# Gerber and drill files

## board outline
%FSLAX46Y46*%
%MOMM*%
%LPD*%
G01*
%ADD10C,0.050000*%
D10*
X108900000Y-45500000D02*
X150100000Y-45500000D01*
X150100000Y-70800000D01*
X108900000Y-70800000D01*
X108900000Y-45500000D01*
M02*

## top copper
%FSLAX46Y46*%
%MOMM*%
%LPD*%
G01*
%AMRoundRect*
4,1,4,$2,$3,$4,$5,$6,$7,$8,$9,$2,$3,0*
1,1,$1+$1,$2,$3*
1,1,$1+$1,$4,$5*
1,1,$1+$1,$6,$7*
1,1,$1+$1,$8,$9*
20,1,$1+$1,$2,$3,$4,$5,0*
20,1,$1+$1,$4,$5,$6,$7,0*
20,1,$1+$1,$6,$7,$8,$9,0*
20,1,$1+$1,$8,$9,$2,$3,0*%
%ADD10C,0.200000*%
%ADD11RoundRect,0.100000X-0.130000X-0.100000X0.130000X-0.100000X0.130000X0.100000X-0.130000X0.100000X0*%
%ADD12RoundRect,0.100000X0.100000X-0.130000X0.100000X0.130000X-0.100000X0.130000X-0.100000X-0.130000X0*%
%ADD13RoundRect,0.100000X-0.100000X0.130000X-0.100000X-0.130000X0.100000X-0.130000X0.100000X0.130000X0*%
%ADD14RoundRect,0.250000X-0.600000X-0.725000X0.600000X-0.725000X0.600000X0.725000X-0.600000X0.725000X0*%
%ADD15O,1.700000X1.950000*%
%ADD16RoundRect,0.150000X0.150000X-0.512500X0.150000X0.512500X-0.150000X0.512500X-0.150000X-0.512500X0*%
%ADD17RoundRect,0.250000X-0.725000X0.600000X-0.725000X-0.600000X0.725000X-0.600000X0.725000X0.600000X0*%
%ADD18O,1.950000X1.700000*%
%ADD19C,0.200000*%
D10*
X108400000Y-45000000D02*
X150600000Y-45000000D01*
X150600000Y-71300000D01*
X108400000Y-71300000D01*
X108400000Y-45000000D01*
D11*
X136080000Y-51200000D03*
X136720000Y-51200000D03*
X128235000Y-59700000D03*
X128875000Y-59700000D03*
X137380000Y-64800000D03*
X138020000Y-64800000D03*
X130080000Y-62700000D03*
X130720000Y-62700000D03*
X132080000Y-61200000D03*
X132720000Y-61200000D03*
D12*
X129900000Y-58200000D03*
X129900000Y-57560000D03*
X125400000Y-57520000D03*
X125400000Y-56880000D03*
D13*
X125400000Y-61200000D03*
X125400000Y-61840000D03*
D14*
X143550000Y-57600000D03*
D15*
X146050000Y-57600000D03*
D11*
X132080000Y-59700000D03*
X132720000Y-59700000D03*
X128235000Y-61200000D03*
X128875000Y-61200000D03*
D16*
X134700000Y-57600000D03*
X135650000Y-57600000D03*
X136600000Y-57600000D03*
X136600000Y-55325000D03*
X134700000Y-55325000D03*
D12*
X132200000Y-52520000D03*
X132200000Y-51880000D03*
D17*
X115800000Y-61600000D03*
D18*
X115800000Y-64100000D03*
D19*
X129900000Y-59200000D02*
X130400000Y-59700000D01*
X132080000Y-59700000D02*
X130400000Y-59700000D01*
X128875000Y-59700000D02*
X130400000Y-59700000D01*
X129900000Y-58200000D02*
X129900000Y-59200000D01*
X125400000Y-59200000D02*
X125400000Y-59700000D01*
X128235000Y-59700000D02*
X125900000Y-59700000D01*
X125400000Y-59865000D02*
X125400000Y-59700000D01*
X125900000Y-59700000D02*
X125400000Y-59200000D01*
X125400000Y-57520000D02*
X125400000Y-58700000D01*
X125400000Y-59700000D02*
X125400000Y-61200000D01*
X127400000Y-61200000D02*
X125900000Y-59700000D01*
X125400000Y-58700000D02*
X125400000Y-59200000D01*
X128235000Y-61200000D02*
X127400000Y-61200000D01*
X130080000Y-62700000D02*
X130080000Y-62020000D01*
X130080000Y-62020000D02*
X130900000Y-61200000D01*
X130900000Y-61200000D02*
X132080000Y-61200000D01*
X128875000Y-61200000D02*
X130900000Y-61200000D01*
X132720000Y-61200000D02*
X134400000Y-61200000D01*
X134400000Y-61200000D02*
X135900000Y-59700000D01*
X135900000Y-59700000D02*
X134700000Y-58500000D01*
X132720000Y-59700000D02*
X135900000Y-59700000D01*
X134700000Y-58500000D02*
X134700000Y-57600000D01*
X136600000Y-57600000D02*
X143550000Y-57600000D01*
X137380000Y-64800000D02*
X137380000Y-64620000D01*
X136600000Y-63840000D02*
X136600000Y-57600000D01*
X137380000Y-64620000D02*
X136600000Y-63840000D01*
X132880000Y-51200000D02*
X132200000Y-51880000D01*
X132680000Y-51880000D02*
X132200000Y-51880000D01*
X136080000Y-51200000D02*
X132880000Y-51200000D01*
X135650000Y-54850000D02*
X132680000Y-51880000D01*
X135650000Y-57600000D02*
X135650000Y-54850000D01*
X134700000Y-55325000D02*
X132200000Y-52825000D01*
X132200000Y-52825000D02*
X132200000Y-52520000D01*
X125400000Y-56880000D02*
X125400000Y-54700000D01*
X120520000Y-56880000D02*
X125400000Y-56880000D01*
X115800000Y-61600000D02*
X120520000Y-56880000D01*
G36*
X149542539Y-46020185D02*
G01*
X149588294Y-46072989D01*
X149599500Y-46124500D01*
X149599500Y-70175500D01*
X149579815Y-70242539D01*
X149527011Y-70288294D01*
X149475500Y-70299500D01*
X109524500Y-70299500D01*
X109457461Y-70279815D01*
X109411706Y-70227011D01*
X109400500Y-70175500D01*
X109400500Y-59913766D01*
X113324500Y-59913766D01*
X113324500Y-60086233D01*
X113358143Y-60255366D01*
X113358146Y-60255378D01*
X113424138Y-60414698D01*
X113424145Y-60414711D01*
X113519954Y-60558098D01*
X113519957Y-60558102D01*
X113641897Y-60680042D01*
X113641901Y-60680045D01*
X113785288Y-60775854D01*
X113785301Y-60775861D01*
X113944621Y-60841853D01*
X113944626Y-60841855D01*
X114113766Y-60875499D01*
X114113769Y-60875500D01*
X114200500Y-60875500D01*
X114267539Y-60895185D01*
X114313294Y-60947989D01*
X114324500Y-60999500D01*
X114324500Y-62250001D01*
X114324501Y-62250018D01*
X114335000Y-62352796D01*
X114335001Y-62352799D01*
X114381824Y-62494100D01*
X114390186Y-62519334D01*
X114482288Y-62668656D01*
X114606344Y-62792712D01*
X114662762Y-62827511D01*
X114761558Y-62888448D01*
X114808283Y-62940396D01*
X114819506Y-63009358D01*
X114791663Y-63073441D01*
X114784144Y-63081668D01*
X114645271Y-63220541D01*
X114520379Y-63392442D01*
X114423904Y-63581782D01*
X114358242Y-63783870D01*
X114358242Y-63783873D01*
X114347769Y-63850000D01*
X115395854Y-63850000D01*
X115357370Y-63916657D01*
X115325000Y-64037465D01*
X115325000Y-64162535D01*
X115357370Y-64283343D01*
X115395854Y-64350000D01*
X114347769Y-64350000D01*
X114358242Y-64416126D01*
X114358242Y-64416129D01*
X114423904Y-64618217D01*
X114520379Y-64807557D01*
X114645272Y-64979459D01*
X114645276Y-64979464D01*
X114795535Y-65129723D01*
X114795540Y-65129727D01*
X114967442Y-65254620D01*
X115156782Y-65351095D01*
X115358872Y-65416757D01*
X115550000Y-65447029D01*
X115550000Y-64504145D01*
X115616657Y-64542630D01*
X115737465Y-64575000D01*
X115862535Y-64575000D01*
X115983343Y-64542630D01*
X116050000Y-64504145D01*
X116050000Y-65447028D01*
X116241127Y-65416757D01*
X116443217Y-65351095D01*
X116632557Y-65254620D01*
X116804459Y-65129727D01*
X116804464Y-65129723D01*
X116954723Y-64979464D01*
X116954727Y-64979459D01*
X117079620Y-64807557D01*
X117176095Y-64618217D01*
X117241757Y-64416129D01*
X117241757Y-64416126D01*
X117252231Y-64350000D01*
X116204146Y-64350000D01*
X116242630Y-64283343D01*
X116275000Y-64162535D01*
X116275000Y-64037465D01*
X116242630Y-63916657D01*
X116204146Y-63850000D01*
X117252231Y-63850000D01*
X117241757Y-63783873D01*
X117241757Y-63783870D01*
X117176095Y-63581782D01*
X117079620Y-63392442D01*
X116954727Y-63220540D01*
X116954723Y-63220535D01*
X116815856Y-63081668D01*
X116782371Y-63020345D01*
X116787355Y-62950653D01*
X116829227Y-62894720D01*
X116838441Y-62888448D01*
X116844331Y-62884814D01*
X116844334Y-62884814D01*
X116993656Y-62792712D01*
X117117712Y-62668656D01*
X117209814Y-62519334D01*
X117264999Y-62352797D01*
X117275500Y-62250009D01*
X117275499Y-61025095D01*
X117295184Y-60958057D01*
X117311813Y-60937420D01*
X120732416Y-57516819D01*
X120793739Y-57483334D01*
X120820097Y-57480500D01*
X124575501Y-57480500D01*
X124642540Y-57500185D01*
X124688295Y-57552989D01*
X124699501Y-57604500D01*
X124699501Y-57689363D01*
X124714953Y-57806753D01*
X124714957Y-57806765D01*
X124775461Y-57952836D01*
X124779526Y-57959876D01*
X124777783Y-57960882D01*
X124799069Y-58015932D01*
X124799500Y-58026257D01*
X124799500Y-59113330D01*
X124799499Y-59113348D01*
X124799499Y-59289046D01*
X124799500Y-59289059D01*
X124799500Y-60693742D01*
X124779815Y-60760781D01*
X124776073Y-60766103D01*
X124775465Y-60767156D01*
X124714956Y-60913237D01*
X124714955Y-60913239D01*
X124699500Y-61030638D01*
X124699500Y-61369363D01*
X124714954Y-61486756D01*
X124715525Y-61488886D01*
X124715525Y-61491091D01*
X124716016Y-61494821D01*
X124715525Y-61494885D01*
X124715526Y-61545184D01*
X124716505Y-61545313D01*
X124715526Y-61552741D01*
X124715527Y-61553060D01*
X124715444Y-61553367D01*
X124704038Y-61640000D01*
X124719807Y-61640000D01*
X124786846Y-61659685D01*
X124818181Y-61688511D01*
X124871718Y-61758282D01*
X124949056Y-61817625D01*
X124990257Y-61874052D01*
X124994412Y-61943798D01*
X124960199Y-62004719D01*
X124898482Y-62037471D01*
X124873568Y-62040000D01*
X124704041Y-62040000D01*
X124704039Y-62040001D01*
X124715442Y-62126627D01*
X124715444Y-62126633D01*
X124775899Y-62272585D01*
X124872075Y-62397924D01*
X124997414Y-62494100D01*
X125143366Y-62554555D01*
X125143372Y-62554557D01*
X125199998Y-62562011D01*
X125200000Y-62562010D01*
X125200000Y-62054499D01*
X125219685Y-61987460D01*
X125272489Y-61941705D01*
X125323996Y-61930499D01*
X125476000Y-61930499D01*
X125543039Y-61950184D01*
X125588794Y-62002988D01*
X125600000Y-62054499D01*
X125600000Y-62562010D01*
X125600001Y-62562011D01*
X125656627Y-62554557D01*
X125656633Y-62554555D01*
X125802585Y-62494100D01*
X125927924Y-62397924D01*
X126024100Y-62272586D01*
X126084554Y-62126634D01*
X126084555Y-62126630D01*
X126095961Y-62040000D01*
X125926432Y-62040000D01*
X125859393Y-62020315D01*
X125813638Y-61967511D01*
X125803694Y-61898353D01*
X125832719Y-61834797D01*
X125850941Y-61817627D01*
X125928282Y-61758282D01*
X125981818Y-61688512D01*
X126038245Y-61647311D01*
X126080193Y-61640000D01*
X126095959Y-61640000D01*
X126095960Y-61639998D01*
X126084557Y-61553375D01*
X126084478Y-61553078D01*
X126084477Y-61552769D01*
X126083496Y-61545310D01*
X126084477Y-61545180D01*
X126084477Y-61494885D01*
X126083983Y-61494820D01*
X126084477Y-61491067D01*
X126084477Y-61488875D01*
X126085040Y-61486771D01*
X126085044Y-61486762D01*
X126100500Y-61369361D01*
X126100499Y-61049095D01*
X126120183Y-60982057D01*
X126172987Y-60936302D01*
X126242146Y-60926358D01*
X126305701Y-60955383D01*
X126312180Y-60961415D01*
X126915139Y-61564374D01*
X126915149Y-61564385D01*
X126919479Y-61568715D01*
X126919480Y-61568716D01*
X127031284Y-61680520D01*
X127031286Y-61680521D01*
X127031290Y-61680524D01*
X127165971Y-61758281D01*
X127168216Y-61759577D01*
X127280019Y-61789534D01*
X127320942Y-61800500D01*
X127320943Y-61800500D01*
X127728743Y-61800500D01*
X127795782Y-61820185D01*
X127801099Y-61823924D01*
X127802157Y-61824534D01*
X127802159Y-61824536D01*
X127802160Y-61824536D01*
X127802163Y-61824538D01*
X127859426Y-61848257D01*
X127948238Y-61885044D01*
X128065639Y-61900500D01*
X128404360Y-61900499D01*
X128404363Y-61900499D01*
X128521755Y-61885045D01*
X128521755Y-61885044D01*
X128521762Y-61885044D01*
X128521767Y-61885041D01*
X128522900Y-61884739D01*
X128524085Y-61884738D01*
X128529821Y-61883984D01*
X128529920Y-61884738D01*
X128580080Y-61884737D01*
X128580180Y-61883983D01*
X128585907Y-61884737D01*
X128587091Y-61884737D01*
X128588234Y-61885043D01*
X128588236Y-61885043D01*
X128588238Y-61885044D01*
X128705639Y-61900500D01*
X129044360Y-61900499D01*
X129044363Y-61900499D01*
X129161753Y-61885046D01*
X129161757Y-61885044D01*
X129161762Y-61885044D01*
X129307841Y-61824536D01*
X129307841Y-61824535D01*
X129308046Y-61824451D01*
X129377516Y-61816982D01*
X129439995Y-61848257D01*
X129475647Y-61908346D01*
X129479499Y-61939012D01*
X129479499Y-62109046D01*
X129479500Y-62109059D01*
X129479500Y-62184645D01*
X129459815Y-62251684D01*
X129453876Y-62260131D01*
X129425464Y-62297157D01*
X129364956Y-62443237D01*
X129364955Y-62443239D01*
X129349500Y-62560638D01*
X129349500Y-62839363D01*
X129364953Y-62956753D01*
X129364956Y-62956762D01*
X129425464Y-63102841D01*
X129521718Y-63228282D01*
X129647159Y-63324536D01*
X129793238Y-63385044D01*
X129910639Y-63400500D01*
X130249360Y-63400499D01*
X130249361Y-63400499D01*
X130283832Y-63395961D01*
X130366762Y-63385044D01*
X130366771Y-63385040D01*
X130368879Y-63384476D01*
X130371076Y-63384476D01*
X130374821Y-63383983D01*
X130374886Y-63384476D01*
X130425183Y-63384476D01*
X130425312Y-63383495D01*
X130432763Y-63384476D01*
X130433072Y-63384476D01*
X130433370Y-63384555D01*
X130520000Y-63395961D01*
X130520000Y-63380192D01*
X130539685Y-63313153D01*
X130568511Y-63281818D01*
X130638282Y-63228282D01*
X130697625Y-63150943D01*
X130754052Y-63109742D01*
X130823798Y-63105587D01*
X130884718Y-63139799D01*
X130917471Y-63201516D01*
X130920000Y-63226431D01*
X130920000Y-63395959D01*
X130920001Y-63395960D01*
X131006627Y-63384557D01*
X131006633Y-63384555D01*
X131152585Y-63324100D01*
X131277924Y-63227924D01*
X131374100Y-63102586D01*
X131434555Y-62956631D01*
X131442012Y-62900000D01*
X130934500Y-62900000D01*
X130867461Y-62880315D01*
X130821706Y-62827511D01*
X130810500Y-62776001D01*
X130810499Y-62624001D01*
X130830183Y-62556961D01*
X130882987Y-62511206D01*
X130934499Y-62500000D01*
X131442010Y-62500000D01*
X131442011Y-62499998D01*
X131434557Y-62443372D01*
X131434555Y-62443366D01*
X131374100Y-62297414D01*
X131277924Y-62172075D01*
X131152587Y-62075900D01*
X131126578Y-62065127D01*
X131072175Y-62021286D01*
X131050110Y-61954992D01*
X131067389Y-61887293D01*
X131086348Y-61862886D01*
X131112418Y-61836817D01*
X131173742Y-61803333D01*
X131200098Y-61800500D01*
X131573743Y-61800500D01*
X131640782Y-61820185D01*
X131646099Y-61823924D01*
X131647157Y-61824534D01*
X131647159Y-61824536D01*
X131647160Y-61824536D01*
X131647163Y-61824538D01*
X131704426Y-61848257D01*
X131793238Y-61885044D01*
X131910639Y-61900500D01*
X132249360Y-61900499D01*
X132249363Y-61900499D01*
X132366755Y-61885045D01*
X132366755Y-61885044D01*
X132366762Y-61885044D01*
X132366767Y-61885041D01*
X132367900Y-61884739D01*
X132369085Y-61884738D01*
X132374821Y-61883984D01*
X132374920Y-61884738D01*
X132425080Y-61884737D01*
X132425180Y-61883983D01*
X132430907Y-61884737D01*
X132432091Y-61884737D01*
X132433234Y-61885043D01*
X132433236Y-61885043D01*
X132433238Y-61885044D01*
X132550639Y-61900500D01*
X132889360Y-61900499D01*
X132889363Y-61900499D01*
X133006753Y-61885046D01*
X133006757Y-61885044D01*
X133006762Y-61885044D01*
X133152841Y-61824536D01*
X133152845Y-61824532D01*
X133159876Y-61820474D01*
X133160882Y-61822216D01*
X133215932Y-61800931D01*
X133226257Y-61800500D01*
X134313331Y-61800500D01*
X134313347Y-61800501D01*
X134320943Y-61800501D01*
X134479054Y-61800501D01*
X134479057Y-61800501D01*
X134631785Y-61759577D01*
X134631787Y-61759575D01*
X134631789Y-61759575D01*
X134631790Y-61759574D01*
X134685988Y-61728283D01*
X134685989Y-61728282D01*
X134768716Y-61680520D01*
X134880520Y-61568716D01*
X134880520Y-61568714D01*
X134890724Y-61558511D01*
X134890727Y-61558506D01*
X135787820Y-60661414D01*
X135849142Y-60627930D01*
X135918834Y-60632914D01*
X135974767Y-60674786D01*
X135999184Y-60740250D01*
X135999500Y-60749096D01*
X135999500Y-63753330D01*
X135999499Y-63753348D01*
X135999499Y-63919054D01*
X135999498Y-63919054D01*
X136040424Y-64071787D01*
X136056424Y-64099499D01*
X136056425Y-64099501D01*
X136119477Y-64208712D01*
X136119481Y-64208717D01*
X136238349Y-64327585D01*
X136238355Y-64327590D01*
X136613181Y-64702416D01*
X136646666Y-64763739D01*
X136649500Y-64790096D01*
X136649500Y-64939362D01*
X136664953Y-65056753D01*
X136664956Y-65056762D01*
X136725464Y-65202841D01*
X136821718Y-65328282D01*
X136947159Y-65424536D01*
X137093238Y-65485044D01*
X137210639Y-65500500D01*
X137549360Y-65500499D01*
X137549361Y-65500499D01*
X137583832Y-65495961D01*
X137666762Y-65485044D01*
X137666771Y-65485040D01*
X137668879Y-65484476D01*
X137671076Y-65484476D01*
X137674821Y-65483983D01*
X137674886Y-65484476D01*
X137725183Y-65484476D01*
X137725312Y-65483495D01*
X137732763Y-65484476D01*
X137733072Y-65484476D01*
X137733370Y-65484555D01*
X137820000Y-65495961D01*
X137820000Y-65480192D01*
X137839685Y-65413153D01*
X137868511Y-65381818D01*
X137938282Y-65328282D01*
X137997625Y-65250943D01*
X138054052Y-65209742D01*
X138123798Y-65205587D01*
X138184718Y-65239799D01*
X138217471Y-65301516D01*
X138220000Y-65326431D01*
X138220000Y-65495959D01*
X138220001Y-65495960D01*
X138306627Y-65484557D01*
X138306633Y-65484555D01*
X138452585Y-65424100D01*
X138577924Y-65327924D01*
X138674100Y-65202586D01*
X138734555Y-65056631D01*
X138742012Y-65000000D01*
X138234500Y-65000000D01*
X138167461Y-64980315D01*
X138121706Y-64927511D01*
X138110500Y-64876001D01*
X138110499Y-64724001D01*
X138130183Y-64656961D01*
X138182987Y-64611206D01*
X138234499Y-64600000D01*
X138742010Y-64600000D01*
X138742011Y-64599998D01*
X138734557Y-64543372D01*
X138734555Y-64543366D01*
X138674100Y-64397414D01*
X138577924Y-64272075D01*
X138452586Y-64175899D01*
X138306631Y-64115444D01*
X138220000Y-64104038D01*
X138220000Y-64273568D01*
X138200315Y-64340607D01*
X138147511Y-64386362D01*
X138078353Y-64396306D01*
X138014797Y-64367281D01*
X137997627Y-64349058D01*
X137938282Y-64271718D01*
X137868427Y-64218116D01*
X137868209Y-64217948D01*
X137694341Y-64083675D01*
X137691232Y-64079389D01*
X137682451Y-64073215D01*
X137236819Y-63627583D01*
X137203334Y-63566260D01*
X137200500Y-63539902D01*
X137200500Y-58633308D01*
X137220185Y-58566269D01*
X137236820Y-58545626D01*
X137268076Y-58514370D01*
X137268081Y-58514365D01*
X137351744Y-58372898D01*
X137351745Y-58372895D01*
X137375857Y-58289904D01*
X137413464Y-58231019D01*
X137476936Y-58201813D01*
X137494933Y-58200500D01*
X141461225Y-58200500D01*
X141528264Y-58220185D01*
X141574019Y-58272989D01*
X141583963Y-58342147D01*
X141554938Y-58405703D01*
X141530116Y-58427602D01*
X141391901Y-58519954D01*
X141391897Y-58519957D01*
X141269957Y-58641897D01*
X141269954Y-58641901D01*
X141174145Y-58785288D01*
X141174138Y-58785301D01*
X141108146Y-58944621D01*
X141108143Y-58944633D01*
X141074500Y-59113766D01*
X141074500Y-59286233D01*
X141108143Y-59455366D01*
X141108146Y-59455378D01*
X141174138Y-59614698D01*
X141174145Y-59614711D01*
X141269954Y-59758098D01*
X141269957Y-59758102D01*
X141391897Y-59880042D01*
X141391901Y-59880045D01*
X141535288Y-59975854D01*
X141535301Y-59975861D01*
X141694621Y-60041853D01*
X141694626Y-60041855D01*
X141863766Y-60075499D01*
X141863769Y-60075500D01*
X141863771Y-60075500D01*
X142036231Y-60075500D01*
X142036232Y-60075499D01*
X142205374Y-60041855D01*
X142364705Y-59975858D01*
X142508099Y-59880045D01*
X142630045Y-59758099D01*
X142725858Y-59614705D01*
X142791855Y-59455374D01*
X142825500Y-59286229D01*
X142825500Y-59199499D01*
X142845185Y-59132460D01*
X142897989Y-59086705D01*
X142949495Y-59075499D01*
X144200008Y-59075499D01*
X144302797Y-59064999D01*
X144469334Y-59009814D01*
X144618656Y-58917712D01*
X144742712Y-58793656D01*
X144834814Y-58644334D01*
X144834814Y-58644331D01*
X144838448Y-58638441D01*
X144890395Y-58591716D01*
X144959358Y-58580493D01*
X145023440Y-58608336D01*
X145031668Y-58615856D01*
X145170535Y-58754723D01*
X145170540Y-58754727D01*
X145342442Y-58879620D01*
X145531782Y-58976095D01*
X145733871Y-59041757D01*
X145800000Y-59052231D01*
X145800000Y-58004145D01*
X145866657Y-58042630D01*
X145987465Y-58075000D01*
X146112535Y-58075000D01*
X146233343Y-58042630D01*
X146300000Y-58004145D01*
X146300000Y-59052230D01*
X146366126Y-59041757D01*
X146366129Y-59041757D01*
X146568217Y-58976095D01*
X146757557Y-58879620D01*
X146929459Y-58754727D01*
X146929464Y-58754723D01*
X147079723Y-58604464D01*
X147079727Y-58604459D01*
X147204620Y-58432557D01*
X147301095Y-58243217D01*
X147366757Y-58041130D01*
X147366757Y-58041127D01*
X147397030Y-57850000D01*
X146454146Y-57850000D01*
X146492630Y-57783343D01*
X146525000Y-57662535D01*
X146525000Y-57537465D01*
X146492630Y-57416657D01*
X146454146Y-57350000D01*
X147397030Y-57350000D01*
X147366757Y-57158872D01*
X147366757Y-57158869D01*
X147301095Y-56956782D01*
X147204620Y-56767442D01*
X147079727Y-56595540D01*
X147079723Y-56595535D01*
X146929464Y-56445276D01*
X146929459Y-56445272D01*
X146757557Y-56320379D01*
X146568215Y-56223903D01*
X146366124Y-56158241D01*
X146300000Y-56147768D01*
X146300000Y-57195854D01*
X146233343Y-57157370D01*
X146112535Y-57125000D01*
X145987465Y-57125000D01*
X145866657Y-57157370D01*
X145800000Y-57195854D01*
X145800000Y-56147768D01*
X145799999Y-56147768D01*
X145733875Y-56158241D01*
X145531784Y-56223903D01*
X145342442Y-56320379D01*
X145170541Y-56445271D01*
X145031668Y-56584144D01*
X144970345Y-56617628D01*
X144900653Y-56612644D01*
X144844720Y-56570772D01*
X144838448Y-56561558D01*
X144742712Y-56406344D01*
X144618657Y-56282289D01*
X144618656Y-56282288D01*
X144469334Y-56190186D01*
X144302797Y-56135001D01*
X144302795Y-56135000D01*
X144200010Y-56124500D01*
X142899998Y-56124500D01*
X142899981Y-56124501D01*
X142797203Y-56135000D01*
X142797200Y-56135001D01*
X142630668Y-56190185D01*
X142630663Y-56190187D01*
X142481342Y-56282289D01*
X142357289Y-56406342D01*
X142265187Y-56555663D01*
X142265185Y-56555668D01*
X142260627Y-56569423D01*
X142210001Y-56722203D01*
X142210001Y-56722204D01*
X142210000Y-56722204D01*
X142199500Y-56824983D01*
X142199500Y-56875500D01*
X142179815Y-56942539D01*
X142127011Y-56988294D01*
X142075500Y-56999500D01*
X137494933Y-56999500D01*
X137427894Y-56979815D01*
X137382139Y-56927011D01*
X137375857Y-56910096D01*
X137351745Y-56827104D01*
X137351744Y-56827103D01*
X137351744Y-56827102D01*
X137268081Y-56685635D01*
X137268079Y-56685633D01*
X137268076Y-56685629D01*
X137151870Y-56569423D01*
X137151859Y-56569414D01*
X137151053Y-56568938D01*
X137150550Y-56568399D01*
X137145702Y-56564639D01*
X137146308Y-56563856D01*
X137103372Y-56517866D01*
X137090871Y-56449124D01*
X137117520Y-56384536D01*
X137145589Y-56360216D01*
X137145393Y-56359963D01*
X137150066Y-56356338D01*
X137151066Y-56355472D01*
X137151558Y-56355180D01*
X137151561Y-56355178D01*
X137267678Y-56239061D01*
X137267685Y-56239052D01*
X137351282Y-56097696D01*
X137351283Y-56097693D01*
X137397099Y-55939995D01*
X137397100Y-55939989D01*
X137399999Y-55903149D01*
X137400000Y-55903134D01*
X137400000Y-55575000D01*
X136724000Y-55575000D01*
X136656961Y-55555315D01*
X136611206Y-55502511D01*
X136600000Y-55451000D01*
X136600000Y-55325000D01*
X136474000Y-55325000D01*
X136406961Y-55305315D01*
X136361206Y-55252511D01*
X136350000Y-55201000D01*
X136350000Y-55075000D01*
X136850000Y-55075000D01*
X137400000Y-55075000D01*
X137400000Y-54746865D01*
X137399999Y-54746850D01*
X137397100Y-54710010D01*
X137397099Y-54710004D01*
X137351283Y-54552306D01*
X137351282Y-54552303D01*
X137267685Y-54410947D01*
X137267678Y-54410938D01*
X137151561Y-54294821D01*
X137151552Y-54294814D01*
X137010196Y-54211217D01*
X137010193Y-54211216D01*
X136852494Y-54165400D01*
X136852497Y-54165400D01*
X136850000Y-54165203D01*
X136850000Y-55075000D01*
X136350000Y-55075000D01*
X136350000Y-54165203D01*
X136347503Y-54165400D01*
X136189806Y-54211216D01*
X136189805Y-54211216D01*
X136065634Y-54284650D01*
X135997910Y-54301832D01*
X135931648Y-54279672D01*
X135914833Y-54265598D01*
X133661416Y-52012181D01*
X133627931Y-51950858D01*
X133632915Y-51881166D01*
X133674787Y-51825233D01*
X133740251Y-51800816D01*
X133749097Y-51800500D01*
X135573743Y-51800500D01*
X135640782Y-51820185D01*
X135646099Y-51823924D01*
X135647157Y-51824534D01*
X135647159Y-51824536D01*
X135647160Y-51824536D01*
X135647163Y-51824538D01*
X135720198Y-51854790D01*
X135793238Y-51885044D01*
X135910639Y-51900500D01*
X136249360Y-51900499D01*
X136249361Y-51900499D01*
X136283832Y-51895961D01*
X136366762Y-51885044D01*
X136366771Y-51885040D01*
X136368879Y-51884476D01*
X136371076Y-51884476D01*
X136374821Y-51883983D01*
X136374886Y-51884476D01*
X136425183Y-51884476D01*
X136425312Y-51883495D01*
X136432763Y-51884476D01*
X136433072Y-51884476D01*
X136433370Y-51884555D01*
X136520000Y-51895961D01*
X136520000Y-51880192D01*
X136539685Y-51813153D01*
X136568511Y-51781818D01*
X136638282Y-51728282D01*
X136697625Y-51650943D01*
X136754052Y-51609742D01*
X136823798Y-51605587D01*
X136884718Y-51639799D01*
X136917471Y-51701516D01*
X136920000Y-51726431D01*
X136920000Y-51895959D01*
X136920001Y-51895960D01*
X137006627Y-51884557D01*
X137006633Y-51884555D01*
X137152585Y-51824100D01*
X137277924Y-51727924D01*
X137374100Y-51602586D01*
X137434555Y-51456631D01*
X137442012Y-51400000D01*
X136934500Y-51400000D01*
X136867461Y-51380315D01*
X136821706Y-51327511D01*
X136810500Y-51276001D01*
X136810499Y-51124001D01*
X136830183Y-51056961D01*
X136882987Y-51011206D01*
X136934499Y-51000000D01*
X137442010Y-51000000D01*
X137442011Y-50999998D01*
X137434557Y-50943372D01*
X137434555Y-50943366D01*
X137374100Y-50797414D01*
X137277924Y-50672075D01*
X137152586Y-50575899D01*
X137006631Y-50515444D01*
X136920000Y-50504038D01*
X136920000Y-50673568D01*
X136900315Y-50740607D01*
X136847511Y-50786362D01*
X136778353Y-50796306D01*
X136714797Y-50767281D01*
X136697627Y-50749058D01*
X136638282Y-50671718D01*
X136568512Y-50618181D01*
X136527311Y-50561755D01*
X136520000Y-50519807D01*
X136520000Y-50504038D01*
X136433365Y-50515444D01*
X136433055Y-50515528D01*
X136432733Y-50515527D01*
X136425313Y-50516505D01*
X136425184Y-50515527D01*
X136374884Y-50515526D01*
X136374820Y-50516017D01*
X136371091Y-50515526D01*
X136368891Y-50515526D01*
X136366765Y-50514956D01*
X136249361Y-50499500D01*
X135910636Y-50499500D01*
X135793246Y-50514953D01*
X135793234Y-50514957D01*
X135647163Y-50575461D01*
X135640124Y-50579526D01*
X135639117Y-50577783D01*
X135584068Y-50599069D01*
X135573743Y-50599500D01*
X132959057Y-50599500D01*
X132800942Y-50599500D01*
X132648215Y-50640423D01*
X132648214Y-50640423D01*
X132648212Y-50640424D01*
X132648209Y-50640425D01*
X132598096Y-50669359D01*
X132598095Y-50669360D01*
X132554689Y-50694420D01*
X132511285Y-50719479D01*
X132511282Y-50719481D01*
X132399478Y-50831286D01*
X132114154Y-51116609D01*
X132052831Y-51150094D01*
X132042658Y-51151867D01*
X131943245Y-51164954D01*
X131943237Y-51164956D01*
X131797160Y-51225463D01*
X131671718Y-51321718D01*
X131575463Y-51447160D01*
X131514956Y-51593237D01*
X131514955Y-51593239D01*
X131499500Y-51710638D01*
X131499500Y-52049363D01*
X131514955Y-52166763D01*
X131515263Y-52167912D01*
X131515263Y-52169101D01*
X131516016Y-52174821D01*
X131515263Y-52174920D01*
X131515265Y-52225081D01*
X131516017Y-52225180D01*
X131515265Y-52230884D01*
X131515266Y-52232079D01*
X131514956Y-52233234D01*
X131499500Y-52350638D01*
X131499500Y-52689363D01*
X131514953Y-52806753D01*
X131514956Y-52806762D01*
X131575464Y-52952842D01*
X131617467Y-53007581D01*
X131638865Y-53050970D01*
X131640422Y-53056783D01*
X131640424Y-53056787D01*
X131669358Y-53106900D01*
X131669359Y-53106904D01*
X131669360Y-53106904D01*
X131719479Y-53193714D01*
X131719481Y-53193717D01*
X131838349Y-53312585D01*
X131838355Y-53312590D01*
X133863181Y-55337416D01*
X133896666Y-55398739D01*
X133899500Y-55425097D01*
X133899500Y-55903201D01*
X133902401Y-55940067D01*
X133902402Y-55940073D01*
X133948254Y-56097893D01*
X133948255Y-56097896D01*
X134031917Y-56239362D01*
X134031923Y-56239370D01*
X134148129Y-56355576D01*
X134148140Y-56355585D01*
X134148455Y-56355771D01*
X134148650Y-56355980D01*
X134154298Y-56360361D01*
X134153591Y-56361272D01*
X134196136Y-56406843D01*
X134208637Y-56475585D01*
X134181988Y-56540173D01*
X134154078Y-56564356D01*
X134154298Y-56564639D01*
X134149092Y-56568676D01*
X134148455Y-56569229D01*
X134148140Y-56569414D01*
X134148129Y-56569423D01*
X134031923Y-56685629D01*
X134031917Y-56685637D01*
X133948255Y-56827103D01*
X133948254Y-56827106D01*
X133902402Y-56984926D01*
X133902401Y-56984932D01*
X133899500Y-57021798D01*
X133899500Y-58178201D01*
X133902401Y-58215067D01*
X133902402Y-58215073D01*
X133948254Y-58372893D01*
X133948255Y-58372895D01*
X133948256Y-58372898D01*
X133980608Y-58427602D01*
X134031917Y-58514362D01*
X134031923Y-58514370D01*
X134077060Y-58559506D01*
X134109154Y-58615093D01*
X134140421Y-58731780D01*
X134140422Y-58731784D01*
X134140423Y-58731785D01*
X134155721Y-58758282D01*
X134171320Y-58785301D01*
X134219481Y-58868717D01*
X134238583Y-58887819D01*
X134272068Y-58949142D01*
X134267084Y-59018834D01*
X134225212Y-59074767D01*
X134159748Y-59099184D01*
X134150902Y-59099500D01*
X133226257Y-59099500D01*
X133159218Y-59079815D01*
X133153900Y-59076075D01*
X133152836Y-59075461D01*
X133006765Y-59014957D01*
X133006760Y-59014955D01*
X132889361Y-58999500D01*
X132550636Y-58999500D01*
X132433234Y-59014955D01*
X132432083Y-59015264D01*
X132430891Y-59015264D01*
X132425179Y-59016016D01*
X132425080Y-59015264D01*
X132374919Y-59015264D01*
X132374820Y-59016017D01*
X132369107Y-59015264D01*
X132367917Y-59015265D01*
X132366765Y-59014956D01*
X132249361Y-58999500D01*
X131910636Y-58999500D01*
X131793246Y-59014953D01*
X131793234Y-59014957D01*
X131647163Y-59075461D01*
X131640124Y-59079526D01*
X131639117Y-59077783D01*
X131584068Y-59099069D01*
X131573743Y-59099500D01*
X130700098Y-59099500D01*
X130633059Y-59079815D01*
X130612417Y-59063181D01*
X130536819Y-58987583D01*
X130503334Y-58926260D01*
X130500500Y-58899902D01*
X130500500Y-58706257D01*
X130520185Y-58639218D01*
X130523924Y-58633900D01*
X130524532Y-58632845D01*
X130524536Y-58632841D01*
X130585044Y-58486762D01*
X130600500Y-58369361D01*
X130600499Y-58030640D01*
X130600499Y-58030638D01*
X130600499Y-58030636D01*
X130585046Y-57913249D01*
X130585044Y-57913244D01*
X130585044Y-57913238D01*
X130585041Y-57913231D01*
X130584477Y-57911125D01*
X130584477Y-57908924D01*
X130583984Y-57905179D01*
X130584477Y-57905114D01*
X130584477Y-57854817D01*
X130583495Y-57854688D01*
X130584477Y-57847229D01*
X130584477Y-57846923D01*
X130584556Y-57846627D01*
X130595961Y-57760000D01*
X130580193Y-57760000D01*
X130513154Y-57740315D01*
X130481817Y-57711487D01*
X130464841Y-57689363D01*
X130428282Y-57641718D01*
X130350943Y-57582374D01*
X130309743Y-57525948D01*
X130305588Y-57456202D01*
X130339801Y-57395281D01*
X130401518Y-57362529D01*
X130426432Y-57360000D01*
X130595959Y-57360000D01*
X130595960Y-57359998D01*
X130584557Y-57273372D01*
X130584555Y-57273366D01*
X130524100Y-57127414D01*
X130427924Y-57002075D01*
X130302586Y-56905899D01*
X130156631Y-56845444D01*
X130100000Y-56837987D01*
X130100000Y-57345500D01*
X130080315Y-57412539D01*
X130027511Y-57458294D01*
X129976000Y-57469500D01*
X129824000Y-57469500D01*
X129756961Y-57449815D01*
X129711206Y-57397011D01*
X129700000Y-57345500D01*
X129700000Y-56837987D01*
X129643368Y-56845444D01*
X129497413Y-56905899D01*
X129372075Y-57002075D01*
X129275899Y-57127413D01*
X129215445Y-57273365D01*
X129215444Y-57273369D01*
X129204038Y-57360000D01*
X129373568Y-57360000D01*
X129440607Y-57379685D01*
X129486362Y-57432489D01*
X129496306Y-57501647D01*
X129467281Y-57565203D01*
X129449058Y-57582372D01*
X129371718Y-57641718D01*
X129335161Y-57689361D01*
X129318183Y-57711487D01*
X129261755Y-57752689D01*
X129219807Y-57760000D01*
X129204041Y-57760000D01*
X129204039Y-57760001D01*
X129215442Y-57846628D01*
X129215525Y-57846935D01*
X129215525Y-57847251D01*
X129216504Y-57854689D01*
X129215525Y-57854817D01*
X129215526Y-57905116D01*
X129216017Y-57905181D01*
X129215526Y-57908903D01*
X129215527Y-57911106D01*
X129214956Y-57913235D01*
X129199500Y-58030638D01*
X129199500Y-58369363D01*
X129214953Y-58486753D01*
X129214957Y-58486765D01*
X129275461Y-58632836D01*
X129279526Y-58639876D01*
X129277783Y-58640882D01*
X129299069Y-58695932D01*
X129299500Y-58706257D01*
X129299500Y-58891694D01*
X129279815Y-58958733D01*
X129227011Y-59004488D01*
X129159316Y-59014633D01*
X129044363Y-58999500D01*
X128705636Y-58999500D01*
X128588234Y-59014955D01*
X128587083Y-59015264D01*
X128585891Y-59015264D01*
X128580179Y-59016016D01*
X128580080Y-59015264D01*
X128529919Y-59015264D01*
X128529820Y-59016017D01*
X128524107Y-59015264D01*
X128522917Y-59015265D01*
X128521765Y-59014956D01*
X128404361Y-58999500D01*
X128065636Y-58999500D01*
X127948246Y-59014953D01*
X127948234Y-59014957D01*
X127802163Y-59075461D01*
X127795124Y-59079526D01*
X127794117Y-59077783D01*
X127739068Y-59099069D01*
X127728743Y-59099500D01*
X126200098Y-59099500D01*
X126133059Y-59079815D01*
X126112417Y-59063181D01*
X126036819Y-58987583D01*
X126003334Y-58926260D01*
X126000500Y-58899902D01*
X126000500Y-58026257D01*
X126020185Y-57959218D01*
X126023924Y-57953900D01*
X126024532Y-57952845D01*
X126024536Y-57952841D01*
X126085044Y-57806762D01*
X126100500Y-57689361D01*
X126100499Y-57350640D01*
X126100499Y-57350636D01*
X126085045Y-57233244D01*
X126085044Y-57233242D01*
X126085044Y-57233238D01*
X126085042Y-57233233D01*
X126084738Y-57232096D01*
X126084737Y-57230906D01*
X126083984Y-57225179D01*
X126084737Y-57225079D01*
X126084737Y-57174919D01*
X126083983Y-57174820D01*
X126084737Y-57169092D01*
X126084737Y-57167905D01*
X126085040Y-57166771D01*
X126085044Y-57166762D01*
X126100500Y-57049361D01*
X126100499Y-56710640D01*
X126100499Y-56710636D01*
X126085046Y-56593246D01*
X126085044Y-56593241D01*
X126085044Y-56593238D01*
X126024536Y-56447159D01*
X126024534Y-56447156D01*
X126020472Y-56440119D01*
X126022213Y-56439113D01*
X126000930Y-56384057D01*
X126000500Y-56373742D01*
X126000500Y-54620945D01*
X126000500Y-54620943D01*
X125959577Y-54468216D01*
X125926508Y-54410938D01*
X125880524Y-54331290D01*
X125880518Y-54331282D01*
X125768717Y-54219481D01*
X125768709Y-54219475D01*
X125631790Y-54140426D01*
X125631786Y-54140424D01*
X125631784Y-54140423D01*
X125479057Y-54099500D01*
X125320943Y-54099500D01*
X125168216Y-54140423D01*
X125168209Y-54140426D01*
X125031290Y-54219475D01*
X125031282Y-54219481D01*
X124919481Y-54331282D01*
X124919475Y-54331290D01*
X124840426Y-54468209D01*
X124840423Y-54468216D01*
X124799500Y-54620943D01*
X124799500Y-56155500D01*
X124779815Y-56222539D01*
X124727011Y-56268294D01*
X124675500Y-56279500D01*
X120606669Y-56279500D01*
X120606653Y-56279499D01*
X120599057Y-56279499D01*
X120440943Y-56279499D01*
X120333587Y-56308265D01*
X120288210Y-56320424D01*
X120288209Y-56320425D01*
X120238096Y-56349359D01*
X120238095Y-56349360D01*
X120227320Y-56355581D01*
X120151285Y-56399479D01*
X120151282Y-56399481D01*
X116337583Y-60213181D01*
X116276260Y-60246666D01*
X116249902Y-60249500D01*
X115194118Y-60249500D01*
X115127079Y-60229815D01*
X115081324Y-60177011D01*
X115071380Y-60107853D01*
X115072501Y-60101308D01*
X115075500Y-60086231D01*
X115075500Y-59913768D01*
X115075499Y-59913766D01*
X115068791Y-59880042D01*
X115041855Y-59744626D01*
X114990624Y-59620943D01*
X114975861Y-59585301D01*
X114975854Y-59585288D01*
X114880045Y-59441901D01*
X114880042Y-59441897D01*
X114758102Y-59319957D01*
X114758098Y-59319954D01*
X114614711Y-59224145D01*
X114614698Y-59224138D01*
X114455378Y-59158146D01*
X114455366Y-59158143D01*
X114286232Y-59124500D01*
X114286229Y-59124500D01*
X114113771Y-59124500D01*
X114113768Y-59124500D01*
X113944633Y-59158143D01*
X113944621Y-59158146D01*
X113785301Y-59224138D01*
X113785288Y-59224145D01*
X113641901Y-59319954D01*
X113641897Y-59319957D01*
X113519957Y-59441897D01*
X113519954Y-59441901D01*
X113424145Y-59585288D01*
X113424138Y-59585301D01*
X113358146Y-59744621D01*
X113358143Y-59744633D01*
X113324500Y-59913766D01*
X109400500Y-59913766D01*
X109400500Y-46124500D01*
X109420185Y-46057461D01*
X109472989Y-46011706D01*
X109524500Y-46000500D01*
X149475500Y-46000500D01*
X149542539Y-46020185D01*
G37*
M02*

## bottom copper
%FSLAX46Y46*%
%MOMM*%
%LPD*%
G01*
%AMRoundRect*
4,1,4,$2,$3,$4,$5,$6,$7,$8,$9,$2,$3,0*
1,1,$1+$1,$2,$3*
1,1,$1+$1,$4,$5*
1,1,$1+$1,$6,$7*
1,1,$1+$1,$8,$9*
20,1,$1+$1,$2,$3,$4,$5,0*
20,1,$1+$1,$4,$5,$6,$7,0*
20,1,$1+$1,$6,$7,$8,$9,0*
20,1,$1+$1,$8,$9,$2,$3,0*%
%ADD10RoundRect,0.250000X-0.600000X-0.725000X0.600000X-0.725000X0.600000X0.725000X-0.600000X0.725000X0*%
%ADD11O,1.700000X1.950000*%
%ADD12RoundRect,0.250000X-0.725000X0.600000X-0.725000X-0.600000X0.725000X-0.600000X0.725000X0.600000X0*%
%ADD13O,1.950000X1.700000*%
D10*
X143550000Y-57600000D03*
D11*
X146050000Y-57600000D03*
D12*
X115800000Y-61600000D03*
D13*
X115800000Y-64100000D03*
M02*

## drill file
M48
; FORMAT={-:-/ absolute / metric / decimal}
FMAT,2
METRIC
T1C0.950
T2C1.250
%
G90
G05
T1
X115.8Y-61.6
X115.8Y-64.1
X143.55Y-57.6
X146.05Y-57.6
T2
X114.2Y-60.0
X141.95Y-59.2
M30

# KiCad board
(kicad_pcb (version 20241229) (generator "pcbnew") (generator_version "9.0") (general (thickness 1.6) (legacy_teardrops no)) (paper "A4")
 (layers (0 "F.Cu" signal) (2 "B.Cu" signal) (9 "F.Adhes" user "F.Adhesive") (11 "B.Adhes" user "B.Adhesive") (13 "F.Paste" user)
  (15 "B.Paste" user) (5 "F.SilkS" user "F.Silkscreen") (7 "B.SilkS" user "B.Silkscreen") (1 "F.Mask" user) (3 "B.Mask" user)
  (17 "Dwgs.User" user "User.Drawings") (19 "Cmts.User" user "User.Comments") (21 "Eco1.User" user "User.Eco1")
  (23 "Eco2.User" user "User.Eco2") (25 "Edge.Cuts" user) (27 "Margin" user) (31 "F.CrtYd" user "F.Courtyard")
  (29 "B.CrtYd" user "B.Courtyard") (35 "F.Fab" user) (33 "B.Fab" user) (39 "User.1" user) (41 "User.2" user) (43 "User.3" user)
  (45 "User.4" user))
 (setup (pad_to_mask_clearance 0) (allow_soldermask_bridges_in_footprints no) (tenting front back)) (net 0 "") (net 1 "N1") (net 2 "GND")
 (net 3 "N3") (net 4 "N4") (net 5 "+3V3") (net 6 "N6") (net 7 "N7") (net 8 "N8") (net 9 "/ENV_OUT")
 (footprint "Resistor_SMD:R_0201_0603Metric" (layer "F.Cu") (at 136.4 51.2)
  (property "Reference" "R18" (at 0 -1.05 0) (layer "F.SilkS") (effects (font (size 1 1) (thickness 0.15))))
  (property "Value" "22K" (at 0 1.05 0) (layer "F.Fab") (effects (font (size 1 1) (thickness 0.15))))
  (pad "" smd roundrect (at -0.345 0) (size 0.318 0.36) (layers "F.Paste") (roundrect_rratio 0.25))
  (pad "" smd roundrect (at 0.345 0) (size 0.318 0.36) (layers "F.Paste") (roundrect_rratio 0.25))
  (pad "1" smd roundrect (at -0.32 0) (size 0.46 0.4) (layers "F.Cu" "F.Mask") (roundrect_rratio 0.25) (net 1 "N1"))
  (pad "2" smd roundrect (at 0.32 0) (size 0.46 0.4) (layers "F.Cu" "F.Mask") (roundrect_rratio 0.25) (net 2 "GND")))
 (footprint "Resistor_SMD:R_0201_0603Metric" (layer "F.Cu") (at 128.555 59.7)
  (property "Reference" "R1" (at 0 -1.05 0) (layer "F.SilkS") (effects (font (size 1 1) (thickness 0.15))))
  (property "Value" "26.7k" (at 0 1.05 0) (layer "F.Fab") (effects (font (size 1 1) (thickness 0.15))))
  (pad "" smd roundrect (at -0.345 0) (size 0.318 0.36) (layers "F.Paste") (roundrect_rratio 0.25))
  (pad "" smd roundrect (at 0.345 0) (size 0.318 0.36) (layers "F.Paste") (roundrect_rratio 0.25))
  (pad "1" smd roundrect (at -0.32 0) (size 0.46 0.4) (layers "F.Cu" "F.Mask") (roundrect_rratio 0.25) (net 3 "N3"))
  (pad "2" smd roundrect (at 0.32 0) (size 0.46 0.4) (layers "F.Cu" "F.Mask") (roundrect_rratio 0.25) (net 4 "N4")))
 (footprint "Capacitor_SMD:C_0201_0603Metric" (layer "F.Cu") (at 137.7 64.8)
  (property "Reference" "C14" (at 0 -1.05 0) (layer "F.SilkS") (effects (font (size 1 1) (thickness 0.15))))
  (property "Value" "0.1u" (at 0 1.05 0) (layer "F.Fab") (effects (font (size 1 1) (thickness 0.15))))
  (pad "" smd roundrect (at -0.345 0) (size 0.318 0.36) (layers "F.Paste") (roundrect_rratio 0.25))
  (pad "" smd roundrect (at 0.345 0) (size 0.318 0.36) (layers "F.Paste") (roundrect_rratio 0.25))
  (pad "1" smd roundrect (at -0.32 0) (size 0.46 0.4) (layers "F.Cu" "F.Mask") (roundrect_rratio 0.25) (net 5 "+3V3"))
  (pad "2" smd roundrect (at 0.32 0) (size 0.46 0.4) (layers "F.Cu" "F.Mask") (roundrect_rratio 0.25) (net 2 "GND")))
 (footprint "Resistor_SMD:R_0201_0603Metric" (layer "F.Cu") (at 130.4 62.7)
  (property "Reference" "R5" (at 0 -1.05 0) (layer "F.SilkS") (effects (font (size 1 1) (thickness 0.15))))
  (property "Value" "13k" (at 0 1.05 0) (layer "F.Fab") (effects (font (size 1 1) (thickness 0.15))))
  (pad "" smd roundrect (at -0.345 0) (size 0.318 0.36) (layers "F.Paste") (roundrect_rratio 0.25))
  (pad "" smd roundrect (at 0.345 0) (size 0.318 0.36) (layers "F.Paste") (roundrect_rratio 0.25))
  (pad "1" smd roundrect (at -0.32 0) (size 0.46 0.4) (layers "F.Cu" "F.Mask") (roundrect_rratio 0.25) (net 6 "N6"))
  (pad "2" smd roundrect (at 0.32 0) (size 0.46 0.4) (layers "F.Cu" "F.Mask") (roundrect_rratio 0.25) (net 2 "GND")))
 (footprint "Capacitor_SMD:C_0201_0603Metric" (layer "F.Cu") (at 132.4 61.2)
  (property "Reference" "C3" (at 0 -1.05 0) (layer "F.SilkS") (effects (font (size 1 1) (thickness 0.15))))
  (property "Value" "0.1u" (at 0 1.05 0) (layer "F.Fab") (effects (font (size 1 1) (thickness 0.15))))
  (pad "" smd roundrect (at -0.345 0) (size 0.318 0.36) (layers "F.Paste") (roundrect_rratio 0.25))
  (pad "" smd roundrect (at 0.345 0) (size 0.318 0.36) (layers "F.Paste") (roundrect_rratio 0.25))
  (pad "1" smd roundrect (at -0.32 0) (size 0.46 0.4) (layers "F.Cu" "F.Mask") (roundrect_rratio 0.25) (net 6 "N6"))
  (pad "2" smd roundrect (at 0.32 0) (size 0.46 0.4) (layers "F.Cu" "F.Mask") (roundrect_rratio 0.25) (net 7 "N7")))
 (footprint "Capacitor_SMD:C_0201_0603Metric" (layer "F.Cu") (at 129.9 57.88 90)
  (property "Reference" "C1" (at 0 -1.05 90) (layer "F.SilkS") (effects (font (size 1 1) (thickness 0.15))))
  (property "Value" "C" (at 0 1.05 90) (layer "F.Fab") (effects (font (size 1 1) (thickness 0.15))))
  (pad "" smd roundrect (at -0.345 0 90) (size 0.318 0.36) (layers "F.Paste") (roundrect_rratio 0.25))
  (pad "" smd roundrect (at 0.345 0 90) (size 0.318 0.36) (layers "F.Paste") (roundrect_rratio 0.25))
  (pad "1" smd roundrect (at -0.32 0 90) (size 0.46 0.4) (layers "F.Cu" "F.Mask") (roundrect_rratio 0.25) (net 4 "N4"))
  (pad "2" smd roundrect (at 0.32 0 90) (size 0.46 0.4) (layers "F.Cu" "F.Mask") (roundrect_rratio 0.25) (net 2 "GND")))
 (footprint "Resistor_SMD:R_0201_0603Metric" (layer "F.Cu") (at 125.4 57.2 90)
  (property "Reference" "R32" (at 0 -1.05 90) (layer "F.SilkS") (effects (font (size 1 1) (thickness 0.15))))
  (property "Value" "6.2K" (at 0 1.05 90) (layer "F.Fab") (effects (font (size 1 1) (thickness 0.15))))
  (pad "" smd roundrect (at -0.345 0 90) (size 0.318 0.36) (layers "F.Paste") (roundrect_rratio 0.25))
  (pad "" smd roundrect (at 0.345 0 90) (size 0.318 0.36) (layers "F.Paste") (roundrect_rratio 0.25))
  (pad "1" smd roundrect (at -0.32 0 90) (size 0.46 0.4) (layers "F.Cu" "F.Mask") (roundrect_rratio 0.25) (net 3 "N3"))
  (pad "2" smd roundrect (at 0.32 0 90) (size 0.46 0.4) (layers "F.Cu" "F.Mask") (roundrect_rratio 0.25) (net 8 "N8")))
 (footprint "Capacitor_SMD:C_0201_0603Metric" (layer "F.Cu") (at 125.4 61.52 -90)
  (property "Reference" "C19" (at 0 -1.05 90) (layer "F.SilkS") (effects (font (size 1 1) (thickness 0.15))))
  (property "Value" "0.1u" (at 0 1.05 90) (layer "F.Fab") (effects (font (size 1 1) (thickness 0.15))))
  (pad "" smd roundrect (at -0.345 0 270) (size 0.318 0.36) (layers "F.Paste") (roundrect_rratio 0.25))
  (pad "" smd roundrect (at 0.345 0 270) (size 0.318 0.36) (layers "F.Paste") (roundrect_rratio 0.25))
  (pad "1" smd roundrect (at -0.32 0 270) (size 0.46 0.4) (layers "F.Cu" "F.Mask") (roundrect_rratio 0.25) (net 3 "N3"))
  (pad "2" smd roundrect (at 0.32 0 270) (size 0.46 0.4) (layers "F.Cu" "F.Mask") (roundrect_rratio 0.25) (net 2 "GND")))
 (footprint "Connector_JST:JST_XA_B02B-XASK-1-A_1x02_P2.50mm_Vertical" (layer "F.Cu") (at 143.55 57.6)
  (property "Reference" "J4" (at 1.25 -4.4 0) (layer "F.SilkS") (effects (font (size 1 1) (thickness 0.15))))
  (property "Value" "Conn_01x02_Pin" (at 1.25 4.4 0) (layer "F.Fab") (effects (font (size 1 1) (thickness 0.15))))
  (pad "" np_thru_hole circle (at -1.6 1.6) (size 1.25 1.25) (drill 1.25) (layers "*.Cu" "*.Mask"))
  (pad "1" thru_hole roundrect (at 0 0) (size 1.7 1.95) (drill 0.95) (layers "*.Cu" "*.Mask") (remove_unused_layers no)
   (roundrect_rratio 0.147059) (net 5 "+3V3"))
  (pad "2" thru_hole oval (at 2.5 0) (size 1.7 1.95) (drill 0.95) (layers "*.Cu" "*.Mask") (remove_unused_layers no) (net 2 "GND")))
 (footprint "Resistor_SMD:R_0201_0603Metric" (layer "F.Cu") (at 132.4 59.7)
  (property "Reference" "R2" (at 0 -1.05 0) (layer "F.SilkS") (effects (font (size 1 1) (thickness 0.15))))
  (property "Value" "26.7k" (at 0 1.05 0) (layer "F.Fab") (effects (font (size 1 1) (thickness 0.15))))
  (pad "" smd roundrect (at -0.345 0) (size 0.318 0.36) (layers "F.Paste") (roundrect_rratio 0.25))
  (pad "" smd roundrect (at 0.345 0) (size 0.318 0.36) (layers "F.Paste") (roundrect_rratio 0.25))
  (pad "1" smd roundrect (at -0.32 0) (size 0.46 0.4) (layers "F.Cu" "F.Mask") (roundrect_rratio 0.25) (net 4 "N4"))
  (pad "2" smd roundrect (at 0.32 0) (size 0.46 0.4) (layers "F.Cu" "F.Mask") (roundrect_rratio 0.25) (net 7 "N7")))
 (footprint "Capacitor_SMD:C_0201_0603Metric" (layer "F.Cu") (at 128.555 61.2)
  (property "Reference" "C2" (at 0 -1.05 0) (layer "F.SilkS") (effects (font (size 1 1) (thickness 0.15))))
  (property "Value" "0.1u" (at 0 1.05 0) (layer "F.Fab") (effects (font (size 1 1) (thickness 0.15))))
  (pad "" smd roundrect (at -0.345 0) (size 0.318 0.36) (layers "F.Paste") (roundrect_rratio 0.25))
  (pad "" smd roundrect (at 0.345 0) (size 0.318 0.36) (layers "F.Paste") (roundrect_rratio 0.25))
  (pad "1" smd roundrect (at -0.32 0) (size 0.46 0.4) (layers "F.Cu" "F.Mask") (roundrect_rratio 0.25) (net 3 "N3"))
  (pad "2" smd roundrect (at 0.32 0) (size 0.46 0.4) (layers "F.Cu" "F.Mask") (roundrect_rratio 0.25) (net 6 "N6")))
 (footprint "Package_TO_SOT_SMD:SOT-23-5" (layer "F.Cu") (at 135.65 56.4625 90)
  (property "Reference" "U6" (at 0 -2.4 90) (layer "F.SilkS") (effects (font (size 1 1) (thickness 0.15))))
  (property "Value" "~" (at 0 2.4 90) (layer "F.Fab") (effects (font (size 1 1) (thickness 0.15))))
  (pad "1" smd roundrect (at -1.1375 -0.95 90) (size 1.325 0.6) (layers "F.Cu" "F.Mask" "F.Paste") (roundrect_rratio 0.25) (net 7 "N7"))
  (pad "2" smd roundrect (at -1.1375 0 90) (size 1.325 0.6) (layers "F.Cu" "F.Mask" "F.Paste") (roundrect_rratio 0.25) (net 1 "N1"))
  (pad "3" smd roundrect (at -1.1375 0.95 90) (size 1.325 0.6) (layers "F.Cu" "F.Mask" "F.Paste") (roundrect_rratio 0.25) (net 5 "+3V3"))
  (pad "4" smd roundrect (at 1.1375 0.95 90) (size 1.325 0.6) (layers "F.Cu" "F.Mask" "F.Paste") (roundrect_rratio 0.25) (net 2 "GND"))
  (pad "5" smd roundrect (at 1.1375 -0.95 90) (size 1.325 0.6) (layers "F.Cu" "F.Mask" "F.Paste") (roundrect_rratio 0.25) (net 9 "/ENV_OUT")))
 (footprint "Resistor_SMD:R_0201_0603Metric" (layer "F.Cu") (at 132.2 52.2 90)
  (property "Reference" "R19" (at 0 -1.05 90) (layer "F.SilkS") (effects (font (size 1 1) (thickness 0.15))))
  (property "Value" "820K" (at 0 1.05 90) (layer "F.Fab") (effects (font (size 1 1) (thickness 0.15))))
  (pad "" smd roundrect (at -0.345 0 90) (size 0.318 0.36) (layers "F.Paste") (roundrect_rratio 0.25))
  (pad "" smd roundrect (at 0.345 0 90) (size 0.318 0.36) (layers "F.Paste") (roundrect_rratio 0.25))
  (pad "1" smd roundrect (at -0.32 0 90) (size 0.46 0.4) (layers "F.Cu" "F.Mask") (roundrect_rratio 0.25) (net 9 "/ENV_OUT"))
  (pad "2" smd roundrect (at 0.32 0 90) (size 0.46 0.4) (layers "F.Cu" "F.Mask") (roundrect_rratio 0.25) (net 1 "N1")))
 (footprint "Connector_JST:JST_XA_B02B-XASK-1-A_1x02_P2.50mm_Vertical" (layer "F.Cu") (at 115.8 61.6 -90)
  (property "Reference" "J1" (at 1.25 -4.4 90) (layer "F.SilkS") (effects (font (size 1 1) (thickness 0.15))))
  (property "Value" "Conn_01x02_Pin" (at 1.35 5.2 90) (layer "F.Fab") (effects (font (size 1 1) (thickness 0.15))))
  (pad "" np_thru_hole circle (at -1.6 1.6 270) (size 1.25 1.25) (drill 1.25) (layers "*.Cu" "*.Mask"))
  (pad "1" thru_hole roundrect (at 0 0 270) (size 1.7 1.95) (drill 0.95) (layers "*.Cu" "*.Mask") (remove_unused_layers no)
   (roundrect_rratio 0.147059) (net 8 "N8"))
  (pad "2" thru_hole oval (at 2.5 0 270) (size 1.7 1.95) (drill 0.95) (layers "*.Cu" "*.Mask") (remove_unused_layers no) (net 2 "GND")))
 (gr_rect (start 108.4 45) (end 150.6 71.3) (stroke (width 0.2) (type default)) (fill no) (layer "F.Cu"))
 (gr_rect (start 108.9 45.5) (end 150.1 70.8) (stroke (width 0.05) (type default)) (fill no) (layer "Edge.Cuts"))
 (segment (start 129.9 59.2) (end 130.4 59.7) (width 0.2) (layer "F.Cu") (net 4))
 (segment (start 132.08 59.7) (end 130.4 59.7) (width 0.2) (layer "F.Cu") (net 4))
 (segment (start 128.875 59.7) (end 130.4 59.7) (width 0.2) (layer "F.Cu") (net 4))
 (segment (start 129.9 58.2) (end 129.9 59.2) (width 0.2) (layer "F.Cu") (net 4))
 (segment (start 125.4 59.2) (end 125.4 59.7) (width 0.2) (layer "F.Cu") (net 3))
 (segment (start 128.235 59.7) (end 125.9 59.7) (width 0.2) (layer "F.Cu") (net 3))
 (segment (start 125.4 59.865) (end 125.4 59.7) (width 0.2) (layer "F.Cu") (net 3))
 (segment (start 125.9 59.7) (end 125.4 59.2) (width 0.2) (layer "F.Cu") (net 3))
 (segment (start 125.4 57.52) (end 125.4 58.7) (width 0.2) (layer "F.Cu") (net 3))
 (segment (start 125.4 59.7) (end 125.4 61.2) (width 0.2) (layer "F.Cu") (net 3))
 (segment (start 127.4 61.2) (end 125.9 59.7) (width 0.2) (layer "F.Cu") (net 3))
 (segment (start 125.4 58.7) (end 125.4 59.2) (width 0.2) (layer "F.Cu") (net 3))
 (segment (start 128.235 61.2) (end 127.4 61.2) (width 0.2) (layer "F.Cu") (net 3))
 (segment (start 130.08 62.7) (end 130.08 62.02) (width 0.2) (layer "F.Cu") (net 6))
 (segment (start 130.08 62.02) (end 130.9 61.2) (width 0.2) (layer "F.Cu") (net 6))
 (segment (start 130.9 61.2) (end 132.08 61.2) (width 0.2) (layer "F.Cu") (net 6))
 (segment (start 128.875 61.2) (end 130.9 61.2) (width 0.2) (layer "F.Cu") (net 6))
 (segment (start 132.72 61.2) (end 134.4 61.2) (width 0.2) (layer "F.Cu") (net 7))
 (segment (start 134.4 61.2) (end 135.9 59.7) (width 0.2) (layer "F.Cu") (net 7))
 (segment (start 135.9 59.7) (end 134.7 58.5) (width 0.2) (layer "F.Cu") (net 7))
 (segment (start 132.72 59.7) (end 135.9 59.7) (width 0.2) (layer "F.Cu") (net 7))
 (segment (start 134.7 58.5) (end 134.7 57.6) (width 0.2) (layer "F.Cu") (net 7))
 (segment (start 136.6 57.6) (end 143.55 57.6) (width 0.2) (layer "F.Cu") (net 5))
 (segment (start 137.38 64.8) (end 137.38 64.62) (width 0.2) (layer "F.Cu") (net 5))
 (segment (start 136.6 63.84) (end 136.6 57.6) (width 0.2) (layer "F.Cu") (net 5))
 (segment (start 137.38 64.62) (end 136.6 63.84) (width 0.2) (layer "F.Cu") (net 5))
 (segment (start 132.88 51.2) (end 132.2 51.88) (width 0.2) (layer "F.Cu") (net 1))
 (segment (start 132.68 51.88) (end 132.2 51.88) (width 0.2) (layer "F.Cu") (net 1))
 (segment (start 136.08 51.2) (end 132.88 51.2) (width 0.2) (layer "F.Cu") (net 1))
 (segment (start 135.65 54.85) (end 132.68 51.88) (width 0.2) (layer "F.Cu") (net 1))
 (segment (start 135.65 57.6) (end 135.65 54.85) (width 0.2) (layer "F.Cu") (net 1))
 (segment (start 134.7 55.325) (end 132.2 52.825) (width 0.2) (layer "F.Cu") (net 9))
 (segment (start 132.2 52.825) (end 132.2 52.52) (width 0.2) (layer "F.Cu") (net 9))
 (segment (start 125.4 56.88) (end 125.4 54.7) (width 0.2) (layer "F.Cu") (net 8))
 (segment (start 120.52 56.88) (end 125.4 56.88) (width 0.2) (layer "F.Cu") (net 8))
 (segment (start 115.8 61.6) (end 120.52 56.88) (width 0.2) (layer "F.Cu") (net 8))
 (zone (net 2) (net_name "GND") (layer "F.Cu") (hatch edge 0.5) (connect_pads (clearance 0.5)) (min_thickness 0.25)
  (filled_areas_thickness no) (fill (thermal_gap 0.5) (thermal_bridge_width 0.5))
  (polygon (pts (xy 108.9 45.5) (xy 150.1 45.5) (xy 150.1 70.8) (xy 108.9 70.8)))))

